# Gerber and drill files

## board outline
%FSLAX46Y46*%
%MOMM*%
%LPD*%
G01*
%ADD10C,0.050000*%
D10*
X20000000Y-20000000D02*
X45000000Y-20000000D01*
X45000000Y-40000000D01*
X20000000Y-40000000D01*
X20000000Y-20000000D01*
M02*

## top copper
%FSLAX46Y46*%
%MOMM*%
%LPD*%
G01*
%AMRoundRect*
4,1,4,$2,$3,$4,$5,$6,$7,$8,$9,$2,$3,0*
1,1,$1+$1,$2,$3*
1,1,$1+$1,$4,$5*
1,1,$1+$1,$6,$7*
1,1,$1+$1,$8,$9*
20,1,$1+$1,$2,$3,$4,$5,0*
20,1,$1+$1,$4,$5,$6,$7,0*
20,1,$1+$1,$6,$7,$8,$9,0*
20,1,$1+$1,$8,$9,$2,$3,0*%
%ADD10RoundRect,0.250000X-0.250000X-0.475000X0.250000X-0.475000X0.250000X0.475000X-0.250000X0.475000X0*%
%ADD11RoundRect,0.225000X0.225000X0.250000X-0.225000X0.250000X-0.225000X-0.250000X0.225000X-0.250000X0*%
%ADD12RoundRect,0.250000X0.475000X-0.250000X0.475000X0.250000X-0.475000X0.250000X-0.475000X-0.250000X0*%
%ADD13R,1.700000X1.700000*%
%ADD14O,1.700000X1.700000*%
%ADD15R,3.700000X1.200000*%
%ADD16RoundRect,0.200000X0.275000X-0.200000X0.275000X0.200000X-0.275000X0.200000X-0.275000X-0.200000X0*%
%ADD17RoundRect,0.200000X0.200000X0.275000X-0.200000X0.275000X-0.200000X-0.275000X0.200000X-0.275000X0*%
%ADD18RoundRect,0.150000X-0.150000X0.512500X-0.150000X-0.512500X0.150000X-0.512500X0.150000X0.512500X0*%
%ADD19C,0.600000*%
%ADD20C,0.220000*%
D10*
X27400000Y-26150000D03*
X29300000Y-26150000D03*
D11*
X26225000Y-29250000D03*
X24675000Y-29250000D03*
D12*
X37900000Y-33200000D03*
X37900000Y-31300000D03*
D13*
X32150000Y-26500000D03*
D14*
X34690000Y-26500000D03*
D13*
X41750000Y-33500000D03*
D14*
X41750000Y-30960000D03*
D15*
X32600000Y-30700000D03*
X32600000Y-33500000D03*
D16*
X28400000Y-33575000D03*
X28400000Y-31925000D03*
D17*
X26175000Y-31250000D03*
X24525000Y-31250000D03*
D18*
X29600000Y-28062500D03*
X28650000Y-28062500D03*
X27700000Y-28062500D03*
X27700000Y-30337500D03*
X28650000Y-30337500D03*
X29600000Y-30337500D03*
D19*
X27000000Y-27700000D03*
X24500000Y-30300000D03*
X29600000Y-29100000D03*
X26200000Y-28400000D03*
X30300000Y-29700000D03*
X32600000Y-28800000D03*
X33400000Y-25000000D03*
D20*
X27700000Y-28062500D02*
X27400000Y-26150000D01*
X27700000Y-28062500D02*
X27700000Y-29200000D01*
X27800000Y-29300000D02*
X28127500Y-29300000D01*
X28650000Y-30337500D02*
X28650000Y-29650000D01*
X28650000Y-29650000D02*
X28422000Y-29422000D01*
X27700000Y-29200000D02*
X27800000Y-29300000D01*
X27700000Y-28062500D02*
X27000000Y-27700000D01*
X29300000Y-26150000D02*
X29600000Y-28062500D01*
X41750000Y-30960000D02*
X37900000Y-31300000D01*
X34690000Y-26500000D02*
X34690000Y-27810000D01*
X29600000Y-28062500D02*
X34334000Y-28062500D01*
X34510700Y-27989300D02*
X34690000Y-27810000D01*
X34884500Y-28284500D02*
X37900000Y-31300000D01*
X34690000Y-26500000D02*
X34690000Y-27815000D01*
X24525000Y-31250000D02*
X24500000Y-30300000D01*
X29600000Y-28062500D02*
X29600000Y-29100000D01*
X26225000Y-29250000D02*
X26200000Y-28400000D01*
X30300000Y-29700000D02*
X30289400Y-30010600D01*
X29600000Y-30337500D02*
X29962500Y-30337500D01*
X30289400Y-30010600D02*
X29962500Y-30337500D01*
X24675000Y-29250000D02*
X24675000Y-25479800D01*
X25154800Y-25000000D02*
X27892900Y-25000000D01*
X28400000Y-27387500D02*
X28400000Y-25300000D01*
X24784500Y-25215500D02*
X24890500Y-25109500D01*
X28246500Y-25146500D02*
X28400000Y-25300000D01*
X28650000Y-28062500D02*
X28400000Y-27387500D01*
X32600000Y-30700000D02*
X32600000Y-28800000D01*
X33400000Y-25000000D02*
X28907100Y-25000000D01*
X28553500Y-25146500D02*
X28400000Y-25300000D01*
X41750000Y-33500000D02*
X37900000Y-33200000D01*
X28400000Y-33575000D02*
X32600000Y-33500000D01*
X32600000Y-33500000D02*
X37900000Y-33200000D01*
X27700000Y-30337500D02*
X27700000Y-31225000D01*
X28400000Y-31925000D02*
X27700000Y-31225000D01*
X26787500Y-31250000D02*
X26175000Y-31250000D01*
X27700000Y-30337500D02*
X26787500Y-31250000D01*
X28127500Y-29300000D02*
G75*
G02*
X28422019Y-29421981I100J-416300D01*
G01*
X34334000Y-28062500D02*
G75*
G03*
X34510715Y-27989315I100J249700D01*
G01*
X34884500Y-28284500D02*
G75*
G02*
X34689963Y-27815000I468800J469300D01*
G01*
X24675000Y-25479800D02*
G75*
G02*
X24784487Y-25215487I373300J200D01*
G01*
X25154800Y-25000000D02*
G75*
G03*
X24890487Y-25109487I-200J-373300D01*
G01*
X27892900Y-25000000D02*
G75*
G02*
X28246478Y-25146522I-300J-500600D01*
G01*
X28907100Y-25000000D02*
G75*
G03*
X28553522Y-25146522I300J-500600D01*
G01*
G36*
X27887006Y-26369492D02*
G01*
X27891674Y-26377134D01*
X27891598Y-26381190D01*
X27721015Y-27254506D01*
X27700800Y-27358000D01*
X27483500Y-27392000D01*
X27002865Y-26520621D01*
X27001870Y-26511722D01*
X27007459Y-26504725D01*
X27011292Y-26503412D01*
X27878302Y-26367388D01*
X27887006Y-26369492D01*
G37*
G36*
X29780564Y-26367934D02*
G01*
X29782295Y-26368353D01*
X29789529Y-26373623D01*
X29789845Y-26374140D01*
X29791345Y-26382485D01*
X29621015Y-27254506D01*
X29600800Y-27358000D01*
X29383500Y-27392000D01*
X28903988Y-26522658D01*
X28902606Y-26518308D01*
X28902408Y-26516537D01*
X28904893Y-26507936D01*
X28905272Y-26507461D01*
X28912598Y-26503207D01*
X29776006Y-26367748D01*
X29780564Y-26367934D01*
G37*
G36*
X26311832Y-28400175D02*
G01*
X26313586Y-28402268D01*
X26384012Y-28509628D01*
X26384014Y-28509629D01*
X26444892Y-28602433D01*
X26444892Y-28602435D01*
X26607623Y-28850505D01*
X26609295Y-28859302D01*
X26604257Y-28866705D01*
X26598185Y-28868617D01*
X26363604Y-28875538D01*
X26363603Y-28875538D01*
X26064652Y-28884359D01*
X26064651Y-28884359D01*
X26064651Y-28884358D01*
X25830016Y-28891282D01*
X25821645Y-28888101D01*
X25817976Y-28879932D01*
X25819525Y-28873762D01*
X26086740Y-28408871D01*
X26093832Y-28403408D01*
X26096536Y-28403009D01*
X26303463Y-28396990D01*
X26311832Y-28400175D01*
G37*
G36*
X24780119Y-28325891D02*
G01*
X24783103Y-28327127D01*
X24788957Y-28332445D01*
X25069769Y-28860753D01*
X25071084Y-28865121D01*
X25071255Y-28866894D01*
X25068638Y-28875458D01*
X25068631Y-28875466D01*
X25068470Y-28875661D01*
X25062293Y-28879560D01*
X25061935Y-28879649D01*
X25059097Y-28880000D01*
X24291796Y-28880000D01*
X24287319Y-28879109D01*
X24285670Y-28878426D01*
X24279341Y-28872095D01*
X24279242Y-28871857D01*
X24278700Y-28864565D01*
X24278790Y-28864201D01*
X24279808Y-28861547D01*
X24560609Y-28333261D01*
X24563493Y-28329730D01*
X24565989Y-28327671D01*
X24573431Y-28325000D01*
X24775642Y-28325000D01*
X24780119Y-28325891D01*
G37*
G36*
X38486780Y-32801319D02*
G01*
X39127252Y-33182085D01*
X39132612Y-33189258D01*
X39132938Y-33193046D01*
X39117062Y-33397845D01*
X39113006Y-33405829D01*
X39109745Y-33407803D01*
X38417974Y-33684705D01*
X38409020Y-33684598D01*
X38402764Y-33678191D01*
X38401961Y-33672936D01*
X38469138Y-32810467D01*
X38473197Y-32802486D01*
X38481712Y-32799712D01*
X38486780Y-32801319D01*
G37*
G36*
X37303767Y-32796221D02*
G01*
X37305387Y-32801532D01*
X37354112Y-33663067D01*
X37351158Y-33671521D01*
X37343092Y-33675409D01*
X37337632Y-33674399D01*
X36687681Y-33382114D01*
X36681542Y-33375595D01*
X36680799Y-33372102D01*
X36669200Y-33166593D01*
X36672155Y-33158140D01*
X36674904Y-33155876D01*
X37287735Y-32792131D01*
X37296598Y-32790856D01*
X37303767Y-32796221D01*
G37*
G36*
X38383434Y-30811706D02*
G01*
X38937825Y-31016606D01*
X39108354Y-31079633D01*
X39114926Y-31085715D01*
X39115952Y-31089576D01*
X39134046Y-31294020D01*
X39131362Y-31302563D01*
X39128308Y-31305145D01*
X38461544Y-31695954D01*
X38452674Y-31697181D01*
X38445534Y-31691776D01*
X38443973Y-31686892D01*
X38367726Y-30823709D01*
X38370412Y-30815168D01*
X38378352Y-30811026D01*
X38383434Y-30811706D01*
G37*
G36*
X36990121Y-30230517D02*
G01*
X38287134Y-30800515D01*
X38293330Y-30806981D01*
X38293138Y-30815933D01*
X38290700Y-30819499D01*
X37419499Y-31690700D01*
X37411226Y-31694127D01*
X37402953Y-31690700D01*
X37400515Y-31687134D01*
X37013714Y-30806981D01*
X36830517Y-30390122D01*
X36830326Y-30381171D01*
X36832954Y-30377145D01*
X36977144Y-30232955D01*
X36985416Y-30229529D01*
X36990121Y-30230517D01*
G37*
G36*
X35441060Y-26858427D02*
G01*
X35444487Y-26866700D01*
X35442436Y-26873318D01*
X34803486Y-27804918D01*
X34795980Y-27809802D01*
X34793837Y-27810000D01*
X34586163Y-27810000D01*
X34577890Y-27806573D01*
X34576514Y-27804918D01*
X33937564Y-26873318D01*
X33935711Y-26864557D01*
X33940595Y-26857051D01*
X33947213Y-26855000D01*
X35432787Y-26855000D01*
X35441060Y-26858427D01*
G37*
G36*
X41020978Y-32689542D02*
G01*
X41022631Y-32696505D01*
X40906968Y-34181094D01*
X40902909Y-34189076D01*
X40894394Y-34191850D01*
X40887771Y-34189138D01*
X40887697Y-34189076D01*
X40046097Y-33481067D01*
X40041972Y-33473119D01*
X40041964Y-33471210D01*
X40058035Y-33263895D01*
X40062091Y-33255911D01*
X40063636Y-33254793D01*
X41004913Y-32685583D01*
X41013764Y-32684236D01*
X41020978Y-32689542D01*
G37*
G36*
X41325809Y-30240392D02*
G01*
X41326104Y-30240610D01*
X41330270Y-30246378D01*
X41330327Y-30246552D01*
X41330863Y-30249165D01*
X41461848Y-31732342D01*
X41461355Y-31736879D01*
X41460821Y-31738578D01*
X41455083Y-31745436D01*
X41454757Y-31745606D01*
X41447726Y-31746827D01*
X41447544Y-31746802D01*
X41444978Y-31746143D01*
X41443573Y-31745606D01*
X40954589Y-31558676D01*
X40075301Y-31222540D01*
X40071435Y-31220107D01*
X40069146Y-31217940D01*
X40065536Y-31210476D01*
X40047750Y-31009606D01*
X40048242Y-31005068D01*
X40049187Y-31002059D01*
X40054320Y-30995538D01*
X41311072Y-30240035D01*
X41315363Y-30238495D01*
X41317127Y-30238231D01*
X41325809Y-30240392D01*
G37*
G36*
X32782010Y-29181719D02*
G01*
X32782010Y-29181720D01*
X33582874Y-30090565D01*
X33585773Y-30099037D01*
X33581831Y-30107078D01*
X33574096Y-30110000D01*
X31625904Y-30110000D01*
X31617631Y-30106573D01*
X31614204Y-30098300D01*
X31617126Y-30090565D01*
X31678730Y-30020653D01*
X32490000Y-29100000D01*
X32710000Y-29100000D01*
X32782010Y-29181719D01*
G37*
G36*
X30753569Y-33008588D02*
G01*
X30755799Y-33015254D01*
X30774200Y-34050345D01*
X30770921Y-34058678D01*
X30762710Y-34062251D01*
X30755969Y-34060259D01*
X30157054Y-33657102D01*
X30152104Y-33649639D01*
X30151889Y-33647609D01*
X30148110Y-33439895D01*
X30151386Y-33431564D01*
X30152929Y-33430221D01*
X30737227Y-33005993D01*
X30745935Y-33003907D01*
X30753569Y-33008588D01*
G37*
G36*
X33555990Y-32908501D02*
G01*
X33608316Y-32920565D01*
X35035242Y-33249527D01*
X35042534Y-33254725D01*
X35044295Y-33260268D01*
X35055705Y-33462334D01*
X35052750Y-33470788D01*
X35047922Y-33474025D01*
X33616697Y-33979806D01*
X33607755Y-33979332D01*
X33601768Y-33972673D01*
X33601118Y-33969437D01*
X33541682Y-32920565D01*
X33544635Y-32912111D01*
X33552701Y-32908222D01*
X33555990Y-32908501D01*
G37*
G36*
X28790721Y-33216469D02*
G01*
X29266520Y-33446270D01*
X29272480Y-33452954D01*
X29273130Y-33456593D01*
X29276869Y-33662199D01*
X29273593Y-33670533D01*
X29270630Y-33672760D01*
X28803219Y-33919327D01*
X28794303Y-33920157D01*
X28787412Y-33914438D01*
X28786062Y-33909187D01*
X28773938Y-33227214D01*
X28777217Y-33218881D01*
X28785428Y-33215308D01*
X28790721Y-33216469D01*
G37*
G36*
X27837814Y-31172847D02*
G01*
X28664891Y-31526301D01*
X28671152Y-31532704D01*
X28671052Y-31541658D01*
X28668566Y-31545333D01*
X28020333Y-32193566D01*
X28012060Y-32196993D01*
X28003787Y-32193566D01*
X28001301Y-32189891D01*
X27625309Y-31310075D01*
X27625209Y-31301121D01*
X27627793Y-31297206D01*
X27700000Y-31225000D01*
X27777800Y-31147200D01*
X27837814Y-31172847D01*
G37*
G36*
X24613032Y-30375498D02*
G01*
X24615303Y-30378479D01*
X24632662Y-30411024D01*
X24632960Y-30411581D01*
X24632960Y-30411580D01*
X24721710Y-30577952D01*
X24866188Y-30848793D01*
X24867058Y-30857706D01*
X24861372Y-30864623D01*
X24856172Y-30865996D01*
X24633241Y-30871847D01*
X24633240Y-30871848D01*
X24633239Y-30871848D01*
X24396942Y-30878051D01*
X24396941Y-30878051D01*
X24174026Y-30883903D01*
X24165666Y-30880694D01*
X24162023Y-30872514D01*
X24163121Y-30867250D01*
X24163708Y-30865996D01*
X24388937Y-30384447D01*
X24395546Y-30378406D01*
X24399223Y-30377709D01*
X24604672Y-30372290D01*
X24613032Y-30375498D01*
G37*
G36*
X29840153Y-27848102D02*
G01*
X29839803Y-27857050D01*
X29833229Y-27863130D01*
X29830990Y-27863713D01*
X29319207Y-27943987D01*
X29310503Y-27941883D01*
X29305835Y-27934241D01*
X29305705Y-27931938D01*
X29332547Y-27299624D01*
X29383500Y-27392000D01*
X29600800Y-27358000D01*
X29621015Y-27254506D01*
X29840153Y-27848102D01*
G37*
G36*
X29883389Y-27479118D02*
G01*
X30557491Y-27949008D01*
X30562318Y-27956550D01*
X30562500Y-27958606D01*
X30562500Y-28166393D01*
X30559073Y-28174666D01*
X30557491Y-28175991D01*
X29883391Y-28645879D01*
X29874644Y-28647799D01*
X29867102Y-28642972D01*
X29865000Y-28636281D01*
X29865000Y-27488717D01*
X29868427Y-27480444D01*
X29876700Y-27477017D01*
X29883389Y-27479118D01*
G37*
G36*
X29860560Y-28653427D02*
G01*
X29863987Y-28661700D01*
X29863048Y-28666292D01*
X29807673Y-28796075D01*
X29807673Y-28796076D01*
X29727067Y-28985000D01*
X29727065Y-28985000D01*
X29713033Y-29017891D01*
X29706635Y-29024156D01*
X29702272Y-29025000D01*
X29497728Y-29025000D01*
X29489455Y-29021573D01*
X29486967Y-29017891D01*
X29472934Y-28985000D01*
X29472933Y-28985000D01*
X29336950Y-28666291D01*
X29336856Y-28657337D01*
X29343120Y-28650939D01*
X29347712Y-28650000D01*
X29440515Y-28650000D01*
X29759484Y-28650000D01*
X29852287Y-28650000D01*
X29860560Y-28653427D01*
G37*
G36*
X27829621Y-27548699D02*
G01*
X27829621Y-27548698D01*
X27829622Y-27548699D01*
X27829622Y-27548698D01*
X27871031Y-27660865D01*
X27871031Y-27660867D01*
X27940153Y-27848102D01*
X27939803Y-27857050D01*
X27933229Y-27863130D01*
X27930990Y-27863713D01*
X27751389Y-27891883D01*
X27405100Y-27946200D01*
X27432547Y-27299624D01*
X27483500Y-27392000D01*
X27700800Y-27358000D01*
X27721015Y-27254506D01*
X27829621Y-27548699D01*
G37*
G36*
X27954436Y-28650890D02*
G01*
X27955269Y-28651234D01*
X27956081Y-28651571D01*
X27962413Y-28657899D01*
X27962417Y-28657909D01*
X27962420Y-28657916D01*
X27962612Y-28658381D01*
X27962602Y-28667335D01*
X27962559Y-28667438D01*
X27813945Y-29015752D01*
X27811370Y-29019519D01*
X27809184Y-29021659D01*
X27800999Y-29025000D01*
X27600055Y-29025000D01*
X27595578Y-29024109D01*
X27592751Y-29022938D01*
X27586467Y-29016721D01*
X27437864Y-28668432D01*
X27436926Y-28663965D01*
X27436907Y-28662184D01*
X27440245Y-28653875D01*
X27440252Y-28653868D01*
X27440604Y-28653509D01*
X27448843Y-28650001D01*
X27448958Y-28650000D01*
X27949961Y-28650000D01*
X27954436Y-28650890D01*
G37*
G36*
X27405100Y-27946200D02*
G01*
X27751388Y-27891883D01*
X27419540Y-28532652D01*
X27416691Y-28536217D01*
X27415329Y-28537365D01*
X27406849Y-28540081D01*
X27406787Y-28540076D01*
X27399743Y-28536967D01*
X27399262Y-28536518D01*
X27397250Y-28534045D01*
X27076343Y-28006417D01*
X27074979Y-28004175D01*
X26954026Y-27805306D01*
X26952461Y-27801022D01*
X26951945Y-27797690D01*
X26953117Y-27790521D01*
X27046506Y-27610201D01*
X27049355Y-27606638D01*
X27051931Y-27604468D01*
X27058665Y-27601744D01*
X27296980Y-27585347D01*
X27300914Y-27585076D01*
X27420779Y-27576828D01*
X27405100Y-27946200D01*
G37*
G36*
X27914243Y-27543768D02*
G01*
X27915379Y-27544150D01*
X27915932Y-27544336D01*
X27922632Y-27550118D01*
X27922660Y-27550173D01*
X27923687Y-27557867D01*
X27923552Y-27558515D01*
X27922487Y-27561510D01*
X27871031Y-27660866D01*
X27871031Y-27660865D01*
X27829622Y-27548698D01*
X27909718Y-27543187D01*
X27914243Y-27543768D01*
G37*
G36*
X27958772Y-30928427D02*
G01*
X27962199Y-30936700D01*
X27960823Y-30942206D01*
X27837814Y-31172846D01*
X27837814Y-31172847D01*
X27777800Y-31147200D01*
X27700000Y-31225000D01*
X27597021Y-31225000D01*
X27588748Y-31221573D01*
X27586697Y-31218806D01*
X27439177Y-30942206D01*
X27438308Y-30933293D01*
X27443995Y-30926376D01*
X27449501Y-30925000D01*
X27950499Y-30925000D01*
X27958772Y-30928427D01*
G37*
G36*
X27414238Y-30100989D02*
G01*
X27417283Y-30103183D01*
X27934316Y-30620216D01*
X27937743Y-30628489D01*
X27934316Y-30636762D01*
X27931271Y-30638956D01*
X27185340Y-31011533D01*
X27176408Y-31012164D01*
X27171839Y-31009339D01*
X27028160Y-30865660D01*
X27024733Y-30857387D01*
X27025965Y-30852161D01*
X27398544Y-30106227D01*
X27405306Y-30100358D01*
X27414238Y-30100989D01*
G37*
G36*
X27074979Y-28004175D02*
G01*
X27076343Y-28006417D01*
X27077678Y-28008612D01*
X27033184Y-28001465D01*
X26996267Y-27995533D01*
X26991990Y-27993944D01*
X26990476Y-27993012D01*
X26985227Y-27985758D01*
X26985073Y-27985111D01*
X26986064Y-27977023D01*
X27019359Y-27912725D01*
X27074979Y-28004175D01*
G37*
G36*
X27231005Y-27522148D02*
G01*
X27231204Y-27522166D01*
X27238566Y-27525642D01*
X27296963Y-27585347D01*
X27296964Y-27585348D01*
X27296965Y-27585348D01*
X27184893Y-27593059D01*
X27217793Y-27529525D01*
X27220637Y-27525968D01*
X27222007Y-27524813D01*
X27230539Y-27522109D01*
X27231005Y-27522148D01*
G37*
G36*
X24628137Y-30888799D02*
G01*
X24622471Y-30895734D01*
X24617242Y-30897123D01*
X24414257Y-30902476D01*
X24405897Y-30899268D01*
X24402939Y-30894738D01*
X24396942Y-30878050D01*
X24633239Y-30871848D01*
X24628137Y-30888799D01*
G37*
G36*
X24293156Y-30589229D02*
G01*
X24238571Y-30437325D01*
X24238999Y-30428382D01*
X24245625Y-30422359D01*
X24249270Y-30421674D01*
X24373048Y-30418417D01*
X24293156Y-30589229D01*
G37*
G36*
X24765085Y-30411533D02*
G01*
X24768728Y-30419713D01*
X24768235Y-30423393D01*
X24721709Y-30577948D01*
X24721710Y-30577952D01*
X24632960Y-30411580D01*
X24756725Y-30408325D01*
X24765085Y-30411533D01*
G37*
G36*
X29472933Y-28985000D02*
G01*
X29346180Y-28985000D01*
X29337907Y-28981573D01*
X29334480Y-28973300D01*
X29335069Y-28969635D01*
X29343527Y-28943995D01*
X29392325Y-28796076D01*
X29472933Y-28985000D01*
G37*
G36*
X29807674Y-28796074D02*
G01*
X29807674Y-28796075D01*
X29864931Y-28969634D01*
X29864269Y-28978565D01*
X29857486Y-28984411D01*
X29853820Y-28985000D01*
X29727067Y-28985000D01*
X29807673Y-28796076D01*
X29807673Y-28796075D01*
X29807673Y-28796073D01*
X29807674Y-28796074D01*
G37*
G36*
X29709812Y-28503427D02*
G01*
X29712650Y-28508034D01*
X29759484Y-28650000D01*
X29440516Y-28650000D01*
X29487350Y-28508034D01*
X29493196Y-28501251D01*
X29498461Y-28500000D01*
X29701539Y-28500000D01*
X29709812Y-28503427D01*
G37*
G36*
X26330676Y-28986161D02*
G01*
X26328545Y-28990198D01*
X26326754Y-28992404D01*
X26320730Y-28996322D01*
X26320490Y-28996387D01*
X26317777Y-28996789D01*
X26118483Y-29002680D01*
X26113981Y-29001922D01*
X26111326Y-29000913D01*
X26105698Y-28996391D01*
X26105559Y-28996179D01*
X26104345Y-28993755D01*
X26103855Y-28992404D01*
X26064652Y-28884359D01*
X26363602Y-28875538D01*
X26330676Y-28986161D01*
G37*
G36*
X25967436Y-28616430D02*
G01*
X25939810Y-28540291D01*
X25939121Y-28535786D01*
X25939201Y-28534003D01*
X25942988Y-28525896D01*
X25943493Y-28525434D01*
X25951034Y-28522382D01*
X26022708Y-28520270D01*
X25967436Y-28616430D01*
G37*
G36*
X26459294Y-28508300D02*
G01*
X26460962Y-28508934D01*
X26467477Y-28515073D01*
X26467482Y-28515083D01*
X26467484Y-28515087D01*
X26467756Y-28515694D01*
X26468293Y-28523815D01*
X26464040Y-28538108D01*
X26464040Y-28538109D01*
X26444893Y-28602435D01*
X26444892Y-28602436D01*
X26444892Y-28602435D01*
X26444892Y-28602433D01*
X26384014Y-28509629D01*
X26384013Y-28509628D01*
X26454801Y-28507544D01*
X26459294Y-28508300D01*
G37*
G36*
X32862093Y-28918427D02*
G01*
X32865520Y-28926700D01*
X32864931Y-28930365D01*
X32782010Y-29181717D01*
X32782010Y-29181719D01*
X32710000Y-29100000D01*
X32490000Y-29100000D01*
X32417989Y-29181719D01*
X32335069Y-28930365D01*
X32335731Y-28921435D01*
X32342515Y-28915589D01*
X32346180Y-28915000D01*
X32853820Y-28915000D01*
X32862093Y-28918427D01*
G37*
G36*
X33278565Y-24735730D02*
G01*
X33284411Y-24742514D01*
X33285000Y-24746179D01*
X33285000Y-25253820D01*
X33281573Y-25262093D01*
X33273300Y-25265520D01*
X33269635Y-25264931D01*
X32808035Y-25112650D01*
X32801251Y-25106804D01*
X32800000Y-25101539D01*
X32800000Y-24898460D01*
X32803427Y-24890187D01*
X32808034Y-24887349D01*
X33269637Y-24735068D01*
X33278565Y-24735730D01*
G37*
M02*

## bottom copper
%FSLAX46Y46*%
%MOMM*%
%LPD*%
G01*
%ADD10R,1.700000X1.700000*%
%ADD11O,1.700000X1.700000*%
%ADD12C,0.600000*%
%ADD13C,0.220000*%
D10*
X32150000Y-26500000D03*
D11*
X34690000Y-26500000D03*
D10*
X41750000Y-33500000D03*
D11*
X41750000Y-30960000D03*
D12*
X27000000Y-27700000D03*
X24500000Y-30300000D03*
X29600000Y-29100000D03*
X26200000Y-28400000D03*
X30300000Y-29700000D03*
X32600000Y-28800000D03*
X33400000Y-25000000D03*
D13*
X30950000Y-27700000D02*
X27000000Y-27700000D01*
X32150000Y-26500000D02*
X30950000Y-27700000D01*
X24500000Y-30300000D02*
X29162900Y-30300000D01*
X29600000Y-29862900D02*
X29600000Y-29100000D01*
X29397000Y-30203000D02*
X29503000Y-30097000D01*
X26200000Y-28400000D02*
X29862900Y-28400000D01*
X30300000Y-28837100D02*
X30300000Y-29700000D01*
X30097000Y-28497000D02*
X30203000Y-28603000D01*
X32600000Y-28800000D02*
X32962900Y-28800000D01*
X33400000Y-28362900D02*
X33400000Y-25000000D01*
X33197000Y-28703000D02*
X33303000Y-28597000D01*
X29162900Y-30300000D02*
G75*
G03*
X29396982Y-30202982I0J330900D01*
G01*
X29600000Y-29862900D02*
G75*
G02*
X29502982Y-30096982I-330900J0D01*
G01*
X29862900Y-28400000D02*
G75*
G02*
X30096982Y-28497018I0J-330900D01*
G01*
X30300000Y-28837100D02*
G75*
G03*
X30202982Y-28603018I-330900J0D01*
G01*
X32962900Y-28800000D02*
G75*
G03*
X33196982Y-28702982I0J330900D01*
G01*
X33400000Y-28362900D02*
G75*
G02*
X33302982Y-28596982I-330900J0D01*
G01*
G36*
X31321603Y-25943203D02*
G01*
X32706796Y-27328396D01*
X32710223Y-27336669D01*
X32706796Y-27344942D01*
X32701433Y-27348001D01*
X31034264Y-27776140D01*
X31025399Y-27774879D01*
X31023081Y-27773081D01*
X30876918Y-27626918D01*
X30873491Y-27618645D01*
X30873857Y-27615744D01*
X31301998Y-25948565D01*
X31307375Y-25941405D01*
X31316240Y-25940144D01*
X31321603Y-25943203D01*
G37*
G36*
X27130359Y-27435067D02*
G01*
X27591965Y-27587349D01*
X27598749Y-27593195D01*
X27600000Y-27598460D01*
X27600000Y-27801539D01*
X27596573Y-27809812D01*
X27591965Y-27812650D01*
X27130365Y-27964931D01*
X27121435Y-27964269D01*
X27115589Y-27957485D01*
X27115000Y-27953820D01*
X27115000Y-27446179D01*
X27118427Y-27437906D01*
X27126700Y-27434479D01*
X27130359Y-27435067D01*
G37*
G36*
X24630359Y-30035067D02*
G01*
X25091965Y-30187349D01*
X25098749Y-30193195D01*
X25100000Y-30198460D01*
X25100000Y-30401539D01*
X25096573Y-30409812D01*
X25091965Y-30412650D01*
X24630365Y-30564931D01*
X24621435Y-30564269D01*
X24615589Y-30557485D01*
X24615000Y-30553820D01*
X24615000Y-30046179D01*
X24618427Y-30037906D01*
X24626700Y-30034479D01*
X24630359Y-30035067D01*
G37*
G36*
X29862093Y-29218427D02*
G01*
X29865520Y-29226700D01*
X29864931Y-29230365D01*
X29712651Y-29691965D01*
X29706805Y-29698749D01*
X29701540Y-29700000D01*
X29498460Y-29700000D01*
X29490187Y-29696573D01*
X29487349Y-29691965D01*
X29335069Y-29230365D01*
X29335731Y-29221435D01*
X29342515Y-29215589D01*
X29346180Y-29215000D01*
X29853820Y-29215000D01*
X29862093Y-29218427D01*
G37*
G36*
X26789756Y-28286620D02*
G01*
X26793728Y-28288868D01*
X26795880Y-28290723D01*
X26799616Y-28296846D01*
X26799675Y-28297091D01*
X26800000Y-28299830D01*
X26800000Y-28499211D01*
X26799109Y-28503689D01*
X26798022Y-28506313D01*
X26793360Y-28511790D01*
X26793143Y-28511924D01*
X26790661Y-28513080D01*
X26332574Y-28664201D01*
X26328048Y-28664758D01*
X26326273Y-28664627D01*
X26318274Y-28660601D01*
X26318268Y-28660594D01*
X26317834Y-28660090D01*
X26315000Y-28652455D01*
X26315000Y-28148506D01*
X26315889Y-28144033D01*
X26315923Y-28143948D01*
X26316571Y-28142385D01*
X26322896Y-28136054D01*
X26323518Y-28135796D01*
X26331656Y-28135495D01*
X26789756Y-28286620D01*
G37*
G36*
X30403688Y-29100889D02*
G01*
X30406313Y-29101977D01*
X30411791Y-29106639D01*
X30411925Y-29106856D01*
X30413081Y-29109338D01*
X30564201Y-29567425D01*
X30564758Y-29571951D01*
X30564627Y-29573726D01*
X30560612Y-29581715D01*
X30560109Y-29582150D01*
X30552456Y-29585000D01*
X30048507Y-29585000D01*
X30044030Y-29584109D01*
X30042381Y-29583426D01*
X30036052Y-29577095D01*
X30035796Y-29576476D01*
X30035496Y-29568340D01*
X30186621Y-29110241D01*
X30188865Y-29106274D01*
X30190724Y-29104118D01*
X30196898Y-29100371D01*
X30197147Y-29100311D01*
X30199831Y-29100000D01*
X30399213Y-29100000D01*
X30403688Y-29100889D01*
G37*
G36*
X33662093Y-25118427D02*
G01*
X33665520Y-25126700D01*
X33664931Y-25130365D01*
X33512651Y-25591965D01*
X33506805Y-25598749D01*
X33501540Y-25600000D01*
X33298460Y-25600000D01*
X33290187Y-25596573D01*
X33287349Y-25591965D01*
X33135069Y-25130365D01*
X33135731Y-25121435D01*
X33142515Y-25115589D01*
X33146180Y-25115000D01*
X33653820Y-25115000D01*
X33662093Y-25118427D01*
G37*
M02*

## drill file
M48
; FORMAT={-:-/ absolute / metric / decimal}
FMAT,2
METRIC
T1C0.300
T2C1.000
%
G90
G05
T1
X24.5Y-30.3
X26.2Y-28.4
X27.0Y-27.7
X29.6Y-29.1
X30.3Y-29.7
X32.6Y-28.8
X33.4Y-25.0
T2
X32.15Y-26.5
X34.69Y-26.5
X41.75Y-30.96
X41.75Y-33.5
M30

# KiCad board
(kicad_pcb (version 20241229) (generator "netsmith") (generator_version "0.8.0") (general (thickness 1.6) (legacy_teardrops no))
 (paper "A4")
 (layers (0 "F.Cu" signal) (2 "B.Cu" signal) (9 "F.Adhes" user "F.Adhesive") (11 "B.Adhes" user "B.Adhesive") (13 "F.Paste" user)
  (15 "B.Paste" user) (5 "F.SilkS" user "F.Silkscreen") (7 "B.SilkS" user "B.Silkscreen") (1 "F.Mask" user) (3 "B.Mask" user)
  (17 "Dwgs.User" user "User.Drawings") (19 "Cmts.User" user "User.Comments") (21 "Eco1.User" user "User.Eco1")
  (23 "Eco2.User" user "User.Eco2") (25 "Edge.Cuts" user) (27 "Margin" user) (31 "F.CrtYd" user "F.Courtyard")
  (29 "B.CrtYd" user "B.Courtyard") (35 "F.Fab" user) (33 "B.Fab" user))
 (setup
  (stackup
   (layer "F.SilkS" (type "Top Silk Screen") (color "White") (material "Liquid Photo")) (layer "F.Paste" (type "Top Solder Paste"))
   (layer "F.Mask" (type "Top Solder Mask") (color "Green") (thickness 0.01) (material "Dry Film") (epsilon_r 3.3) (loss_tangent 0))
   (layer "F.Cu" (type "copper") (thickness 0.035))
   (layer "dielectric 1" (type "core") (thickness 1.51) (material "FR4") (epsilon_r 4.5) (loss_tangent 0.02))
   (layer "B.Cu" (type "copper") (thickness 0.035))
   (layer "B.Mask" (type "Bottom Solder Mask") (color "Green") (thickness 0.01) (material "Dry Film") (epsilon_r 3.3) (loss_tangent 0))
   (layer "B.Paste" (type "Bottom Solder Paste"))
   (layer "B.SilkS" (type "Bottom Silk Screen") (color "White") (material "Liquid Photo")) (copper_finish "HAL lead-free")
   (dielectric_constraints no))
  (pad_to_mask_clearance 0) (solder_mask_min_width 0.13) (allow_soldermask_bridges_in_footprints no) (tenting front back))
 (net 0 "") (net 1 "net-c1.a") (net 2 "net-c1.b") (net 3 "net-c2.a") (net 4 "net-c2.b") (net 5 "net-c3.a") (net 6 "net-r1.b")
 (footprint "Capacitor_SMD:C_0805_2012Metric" (layer "F.Cu") (at 28.35 26.15)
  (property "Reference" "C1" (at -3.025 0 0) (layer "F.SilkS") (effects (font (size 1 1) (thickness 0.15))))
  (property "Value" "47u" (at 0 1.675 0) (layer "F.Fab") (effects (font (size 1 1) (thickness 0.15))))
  (pad "1" smd roundrect (at -0.95 0) (size 1 1.45) (layers "F.Cu" "F.Mask" "F.Paste") (roundrect_rratio 0.25) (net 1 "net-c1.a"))
  (pad "2" smd roundrect (at 0.95 0) (size 1 1.45) (layers "F.Cu" "F.Mask" "F.Paste") (roundrect_rratio 0.25) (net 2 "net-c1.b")))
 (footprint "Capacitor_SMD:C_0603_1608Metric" (layer "F.Cu") (at 25.45 29.25 180)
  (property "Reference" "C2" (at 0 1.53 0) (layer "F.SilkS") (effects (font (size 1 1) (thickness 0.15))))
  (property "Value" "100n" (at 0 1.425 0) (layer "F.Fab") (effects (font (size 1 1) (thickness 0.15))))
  (pad "1" smd roundrect (at -0.775 0 180) (size 0.9 0.95) (layers "F.Cu" "F.Mask" "F.Paste") (roundrect_rratio 0.25) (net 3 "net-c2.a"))
  (pad "2" smd roundrect (at 0.775 0 180) (size 0.9 0.95) (layers "F.Cu" "F.Mask" "F.Paste") (roundrect_rratio 0.25) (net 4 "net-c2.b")))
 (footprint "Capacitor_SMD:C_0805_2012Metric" (layer "F.Cu") (at 37.9 32.25 90)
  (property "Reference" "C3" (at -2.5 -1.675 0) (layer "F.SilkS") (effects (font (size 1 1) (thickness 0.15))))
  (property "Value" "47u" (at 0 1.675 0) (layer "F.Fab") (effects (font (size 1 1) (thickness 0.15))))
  (pad "1" smd roundrect (at -0.95 0 90) (size 1 1.45) (layers "F.Cu" "F.Mask" "F.Paste") (roundrect_rratio 0.25) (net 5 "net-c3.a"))
  (pad "2" smd roundrect (at 0.95 0 90) (size 1 1.45) (layers "F.Cu" "F.Mask" "F.Paste") (roundrect_rratio 0.25) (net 2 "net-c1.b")))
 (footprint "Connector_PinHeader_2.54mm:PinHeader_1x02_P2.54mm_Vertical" (layer "F.Cu") (at 32.15 26.5 90)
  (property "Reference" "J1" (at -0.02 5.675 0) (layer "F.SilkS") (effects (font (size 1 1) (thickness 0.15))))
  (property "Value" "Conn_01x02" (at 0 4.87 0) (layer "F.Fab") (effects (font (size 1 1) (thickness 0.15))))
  (pad "1" thru_hole rect (at 0 0 90) (size 1.7 1.7) (drill 1) (layers "*.Cu" "*.Mask") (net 1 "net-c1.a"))
  (pad "2" thru_hole oval (at 0 2.54 90) (size 1.7 1.7) (drill 1) (layers "*.Cu" "*.Mask") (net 2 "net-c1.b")))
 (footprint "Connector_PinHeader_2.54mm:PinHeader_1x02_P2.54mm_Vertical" (layer "F.Cu") (at 41.75 33.5 180)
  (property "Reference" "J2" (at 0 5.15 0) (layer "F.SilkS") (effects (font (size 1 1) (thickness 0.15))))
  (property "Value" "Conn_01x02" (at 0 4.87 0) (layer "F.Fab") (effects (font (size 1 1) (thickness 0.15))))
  (pad "1" thru_hole rect (at 0 0 180) (size 1.7 1.7) (drill 1) (layers "*.Cu" "*.Mask") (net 5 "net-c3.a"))
  (pad "2" thru_hole oval (at 0 2.54 180) (size 1.7 1.7) (drill 1) (layers "*.Cu" "*.Mask") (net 2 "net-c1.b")))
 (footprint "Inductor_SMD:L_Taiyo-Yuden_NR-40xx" (layer "F.Cu") (at 32.6 32.1 270)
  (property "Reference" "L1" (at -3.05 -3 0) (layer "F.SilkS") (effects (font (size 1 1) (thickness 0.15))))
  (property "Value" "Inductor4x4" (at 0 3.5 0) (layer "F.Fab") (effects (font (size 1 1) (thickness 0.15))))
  (pad "1" smd rect (at -1.4 0 270) (size 1.2 3.7) (layers "F.Cu" "F.Mask" "F.Paste") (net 4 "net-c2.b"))
  (pad "2" smd rect (at 1.4 0 270) (size 1.2 3.7) (layers "F.Cu" "F.Mask" "F.Paste") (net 5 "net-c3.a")))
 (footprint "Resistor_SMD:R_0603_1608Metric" (layer "F.Cu") (at 28.4 32.75 90)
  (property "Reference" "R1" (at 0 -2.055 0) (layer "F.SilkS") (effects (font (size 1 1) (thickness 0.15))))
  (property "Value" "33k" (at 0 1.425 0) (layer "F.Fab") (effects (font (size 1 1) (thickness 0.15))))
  (pad "1" smd roundrect (at -0.825 0 90) (size 0.8 0.95) (layers "F.Cu" "F.Mask" "F.Paste") (roundrect_rratio 0.25) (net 5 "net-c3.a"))
  (pad "2" smd roundrect (at 0.825 0 90) (size 0.8 0.95) (layers "F.Cu" "F.Mask" "F.Paste") (roundrect_rratio 0.25) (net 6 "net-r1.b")))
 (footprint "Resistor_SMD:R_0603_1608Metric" (layer "F.Cu") (at 25.35 31.25 180)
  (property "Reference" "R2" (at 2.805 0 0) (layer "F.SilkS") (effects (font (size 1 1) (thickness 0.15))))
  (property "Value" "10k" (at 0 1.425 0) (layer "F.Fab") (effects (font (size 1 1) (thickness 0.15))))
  (pad "1" smd roundrect (at -0.825 0 180) (size 0.8 0.95) (layers "F.Cu" "F.Mask" "F.Paste") (roundrect_rratio 0.25) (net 6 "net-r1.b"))
  (pad "2" smd roundrect (at 0.825 0 180) (size 0.8 0.95) (layers "F.Cu" "F.Mask" "F.Paste") (roundrect_rratio 0.25) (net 2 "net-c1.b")))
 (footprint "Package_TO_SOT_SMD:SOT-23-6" (layer "F.Cu") (at 28.65 29.2 270)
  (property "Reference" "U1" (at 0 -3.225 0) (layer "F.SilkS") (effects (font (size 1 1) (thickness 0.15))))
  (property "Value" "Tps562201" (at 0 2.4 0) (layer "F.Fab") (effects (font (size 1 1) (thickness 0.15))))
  (pad "1" smd roundrect (at -1.1375 -0.95 270) (size 1.325 0.6) (layers "F.Cu" "F.Mask" "F.Paste") (roundrect_rratio 0.25)
   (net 2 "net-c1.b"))
  (pad "2" smd roundrect (at -1.1375 0 270) (size 1.325 0.6) (layers "F.Cu" "F.Mask" "F.Paste") (roundrect_rratio 0.25) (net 4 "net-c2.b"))
  (pad "3" smd roundrect (at -1.1375 0.95 270) (size 1.325 0.6) (layers "F.Cu" "F.Mask" "F.Paste") (roundrect_rratio 0.25)
   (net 1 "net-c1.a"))
  (pad "4" smd roundrect (at 1.1375 0.95 270) (size 1.325 0.6) (layers "F.Cu" "F.Mask" "F.Paste") (roundrect_rratio 0.25) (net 6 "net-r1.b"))
  (pad "5" smd roundrect (at 1.1375 0 270) (size 1.325 0.6) (layers "F.Cu" "F.Mask" "F.Paste") (roundrect_rratio 0.25) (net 1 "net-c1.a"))
  (pad "6" smd roundrect (at 1.1375 -0.95 270) (size 1.325 0.6) (layers "F.Cu" "F.Mask" "F.Paste") (roundrect_rratio 0.25)
   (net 3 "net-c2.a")))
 (segment (start 27.7 28.0625) (end 27.4 26.15) (width 0.22) (layer "F.Cu") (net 1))
 (segment (start 27.7 28.0625) (end 27.7 29.2) (width 0.22) (layer "F.Cu") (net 1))
 (segment (start 27.8 29.3) (end 28.1275 29.3) (width 0.22) (layer "F.Cu") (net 1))
 (segment (start 28.65 30.3375) (end 28.65 29.65) (width 0.22) (layer "F.Cu") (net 1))
 (segment (start 28.65 29.65) (end 28.422 29.422) (width 0.22) (layer "F.Cu") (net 1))
 (segment (start 27.7 29.2) (end 27.8 29.3) (width 0.22) (layer "F.Cu") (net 1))
 (segment (start 30.95 27.7) (end 27 27.7) (width 0.22) (layer "B.Cu") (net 1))
 (segment (start 27.7 28.0625) (end 27 27.7) (width 0.22) (layer "F.Cu") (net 1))
 (segment (start 32.15 26.5) (end 30.95 27.7) (width 0.22) (layer "B.Cu") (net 1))
 (segment (start 29.3 26.15) (end 29.6 28.0625) (width 0.22) (layer "F.Cu") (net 2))
 (segment (start 41.75 30.96) (end 37.9 31.3) (width 0.22) (layer "F.Cu") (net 2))
 (segment (start 34.69 26.5) (end 34.69 27.81) (width 0.22) (layer "F.Cu") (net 2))
 (segment (start 29.6 28.0625) (end 34.334 28.0625) (width 0.22) (layer "F.Cu") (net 2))
 (segment (start 34.5107 27.9893) (end 34.69 27.81) (width 0.22) (layer "F.Cu") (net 2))
 (segment (start 34.8845 28.2845) (end 37.9 31.3) (width 0.22) (layer "F.Cu") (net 2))
 (segment (start 34.69 26.5) (end 34.69 27.815) (width 0.22) (layer "F.Cu") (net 2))
 (segment (start 24.525 31.25) (end 24.5 30.3) (width 0.22) (layer "F.Cu") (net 2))
 (segment (start 24.5 30.3) (end 29.1629 30.3) (width 0.22) (layer "B.Cu") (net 2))
 (segment (start 29.6 29.8629) (end 29.6 29.1) (width 0.22) (layer "B.Cu") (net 2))
 (segment (start 29.6 28.0625) (end 29.6 29.1) (width 0.22) (layer "F.Cu") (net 2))
 (segment (start 29.397 30.203) (end 29.503 30.097) (width 0.22) (layer "B.Cu") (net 2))
 (segment (start 26.225 29.25) (end 26.2 28.4) (width 0.22) (layer "F.Cu") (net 3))
 (segment (start 26.2 28.4) (end 29.8629 28.4) (width 0.22) (layer "B.Cu") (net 3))
 (segment (start 30.3 28.8371) (end 30.3 29.7) (width 0.22) (layer "B.Cu") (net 3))
 (segment (start 30.3 29.7) (end 30.2894 30.0106) (width 0.22) (layer "F.Cu") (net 3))
 (segment (start 29.6 30.3375) (end 29.9625 30.3375) (width 0.22) (layer "F.Cu") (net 3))
 (segment (start 30.097 28.497) (end 30.203 28.603) (width 0.22) (layer "B.Cu") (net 3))
 (segment (start 30.2894 30.0106) (end 29.9625 30.3375) (width 0.22) (layer "F.Cu") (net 3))
 (segment (start 24.675 29.25) (end 24.675 25.4798) (width 0.22) (layer "F.Cu") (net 4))
 (segment (start 25.1548 25) (end 27.8929 25) (width 0.22) (layer "F.Cu") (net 4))
 (segment (start 28.4 27.3875) (end 28.4 25.3) (width 0.22) (layer "F.Cu") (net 4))
 (segment (start 24.7845 25.2155) (end 24.8905 25.1095) (width 0.22) (layer "F.Cu") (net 4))
 (segment (start 28.2465 25.1465) (end 28.4 25.3) (width 0.22) (layer "F.Cu") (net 4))
 (segment (start 28.65 28.0625) (end 28.4 27.3875) (width 0.22) (layer "F.Cu") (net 4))
 (segment (start 32.6 30.7) (end 32.6 28.8) (width 0.22) (layer "F.Cu") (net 4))
 (segment (start 32.6 28.8) (end 32.9629 28.8) (width 0.22) (layer "B.Cu") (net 4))
 (segment (start 33.4 28.3629) (end 33.4 25) (width 0.22) (layer "B.Cu") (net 4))
 (segment (start 33.4 25) (end 28.9071 25) (width 0.22) (layer "F.Cu") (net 4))
 (segment (start 33.197 28.703) (end 33.303 28.597) (width 0.22) (layer "B.Cu") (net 4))
 (segment (start 28.5535 25.1465) (end 28.4 25.3) (width 0.22) (layer "F.Cu") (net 4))
 (segment (start 41.75 33.5) (end 37.9 33.2) (width 0.22) (layer "F.Cu") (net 5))
 (segment (start 28.4 33.575) (end 32.6 33.5) (width 0.22) (layer "F.Cu") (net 5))
 (segment (start 32.6 33.5) (end 37.9 33.2) (width 0.22) (layer "F.Cu") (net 5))
 (segment (start 27.7 30.3375) (end 27.7 31.225) (width 0.22) (layer "F.Cu") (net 6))
 (segment (start 28.4 31.925) (end 27.7 31.225) (width 0.22) (layer "F.Cu") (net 6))
 (segment (start 26.7875 31.25) (end 26.175 31.25) (width 0.22) (layer "F.Cu") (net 6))
 (segment (start 27.7 30.3375) (end 26.7875 31.25) (width 0.22) (layer "F.Cu") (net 6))
 (arc (start 28.1275 29.3) (mid 28.2869 29.3317) (end 28.422 29.422) (width 0.22) (layer "F.Cu") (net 1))
 (arc (start 34.334 28.0625) (mid 34.4296 28.0435) (end 34.5107 27.9893) (width 0.22) (layer "F.Cu") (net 2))
 (arc (start 34.8845 28.2845) (mid 34.7405 28.0691) (end 34.69 27.815) (width 0.22) (layer "F.Cu") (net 2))
 (arc (start 29.1629 30.3) (mid 29.2896 30.2748) (end 29.397 30.203) (width 0.22) (layer "B.Cu") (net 2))
 (arc (start 29.6 29.8629) (mid 29.5748 29.9896) (end 29.503 30.097) (width 0.22) (layer "B.Cu") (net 2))
 (arc (start 29.8629 28.4) (mid 29.9896 28.4252) (end 30.097 28.497) (width 0.22) (layer "B.Cu") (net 3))
 (arc (start 30.3 28.8371) (mid 30.2748 28.7104) (end 30.203 28.603) (width 0.22) (layer "B.Cu") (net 3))
 (arc (start 24.675 25.4798) (mid 24.7034 25.3368) (end 24.7845 25.2155) (width 0.22) (layer "F.Cu") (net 4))
 (arc (start 25.1548 25) (mid 25.0118 25.0284) (end 24.8905 25.1095) (width 0.22) (layer "F.Cu") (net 4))
 (arc (start 27.8929 25) (mid 28.0842 25.0381) (end 28.2465 25.1465) (width 0.22) (layer "F.Cu") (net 4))
 (arc (start 32.9629 28.8) (mid 33.0896 28.7748) (end 33.197 28.703) (width 0.22) (layer "B.Cu") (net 4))
 (arc (start 33.4 28.3629) (mid 33.3748 28.4896) (end 33.303 28.597) (width 0.22) (layer "B.Cu") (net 4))
 (arc (start 28.9071 25) (mid 28.7158 25.0381) (end 28.5535 25.1465) (width 0.22) (layer "F.Cu") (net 4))
 (via (at 27 27.7) (size 0.6) (drill 0.3) (layers "F.Cu" "B.Cu") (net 1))
 (via (at 24.5 30.3) (size 0.6) (drill 0.3) (layers "F.Cu" "B.Cu") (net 2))
 (via (at 29.6 29.1) (size 0.6) (drill 0.3) (layers "F.Cu" "B.Cu") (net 2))
 (via (at 26.2 28.4) (size 0.6) (drill 0.3) (layers "F.Cu" "B.Cu") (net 3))
 (via (at 30.3 29.7) (size 0.6) (drill 0.3) (layers "F.Cu" "B.Cu") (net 3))
 (via (at 32.6 28.8) (size 0.6) (drill 0.3) (layers "F.Cu" "B.Cu") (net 4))
 (via (at 33.4 25) (size 0.6) (drill 0.3) (layers "F.Cu" "B.Cu") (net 4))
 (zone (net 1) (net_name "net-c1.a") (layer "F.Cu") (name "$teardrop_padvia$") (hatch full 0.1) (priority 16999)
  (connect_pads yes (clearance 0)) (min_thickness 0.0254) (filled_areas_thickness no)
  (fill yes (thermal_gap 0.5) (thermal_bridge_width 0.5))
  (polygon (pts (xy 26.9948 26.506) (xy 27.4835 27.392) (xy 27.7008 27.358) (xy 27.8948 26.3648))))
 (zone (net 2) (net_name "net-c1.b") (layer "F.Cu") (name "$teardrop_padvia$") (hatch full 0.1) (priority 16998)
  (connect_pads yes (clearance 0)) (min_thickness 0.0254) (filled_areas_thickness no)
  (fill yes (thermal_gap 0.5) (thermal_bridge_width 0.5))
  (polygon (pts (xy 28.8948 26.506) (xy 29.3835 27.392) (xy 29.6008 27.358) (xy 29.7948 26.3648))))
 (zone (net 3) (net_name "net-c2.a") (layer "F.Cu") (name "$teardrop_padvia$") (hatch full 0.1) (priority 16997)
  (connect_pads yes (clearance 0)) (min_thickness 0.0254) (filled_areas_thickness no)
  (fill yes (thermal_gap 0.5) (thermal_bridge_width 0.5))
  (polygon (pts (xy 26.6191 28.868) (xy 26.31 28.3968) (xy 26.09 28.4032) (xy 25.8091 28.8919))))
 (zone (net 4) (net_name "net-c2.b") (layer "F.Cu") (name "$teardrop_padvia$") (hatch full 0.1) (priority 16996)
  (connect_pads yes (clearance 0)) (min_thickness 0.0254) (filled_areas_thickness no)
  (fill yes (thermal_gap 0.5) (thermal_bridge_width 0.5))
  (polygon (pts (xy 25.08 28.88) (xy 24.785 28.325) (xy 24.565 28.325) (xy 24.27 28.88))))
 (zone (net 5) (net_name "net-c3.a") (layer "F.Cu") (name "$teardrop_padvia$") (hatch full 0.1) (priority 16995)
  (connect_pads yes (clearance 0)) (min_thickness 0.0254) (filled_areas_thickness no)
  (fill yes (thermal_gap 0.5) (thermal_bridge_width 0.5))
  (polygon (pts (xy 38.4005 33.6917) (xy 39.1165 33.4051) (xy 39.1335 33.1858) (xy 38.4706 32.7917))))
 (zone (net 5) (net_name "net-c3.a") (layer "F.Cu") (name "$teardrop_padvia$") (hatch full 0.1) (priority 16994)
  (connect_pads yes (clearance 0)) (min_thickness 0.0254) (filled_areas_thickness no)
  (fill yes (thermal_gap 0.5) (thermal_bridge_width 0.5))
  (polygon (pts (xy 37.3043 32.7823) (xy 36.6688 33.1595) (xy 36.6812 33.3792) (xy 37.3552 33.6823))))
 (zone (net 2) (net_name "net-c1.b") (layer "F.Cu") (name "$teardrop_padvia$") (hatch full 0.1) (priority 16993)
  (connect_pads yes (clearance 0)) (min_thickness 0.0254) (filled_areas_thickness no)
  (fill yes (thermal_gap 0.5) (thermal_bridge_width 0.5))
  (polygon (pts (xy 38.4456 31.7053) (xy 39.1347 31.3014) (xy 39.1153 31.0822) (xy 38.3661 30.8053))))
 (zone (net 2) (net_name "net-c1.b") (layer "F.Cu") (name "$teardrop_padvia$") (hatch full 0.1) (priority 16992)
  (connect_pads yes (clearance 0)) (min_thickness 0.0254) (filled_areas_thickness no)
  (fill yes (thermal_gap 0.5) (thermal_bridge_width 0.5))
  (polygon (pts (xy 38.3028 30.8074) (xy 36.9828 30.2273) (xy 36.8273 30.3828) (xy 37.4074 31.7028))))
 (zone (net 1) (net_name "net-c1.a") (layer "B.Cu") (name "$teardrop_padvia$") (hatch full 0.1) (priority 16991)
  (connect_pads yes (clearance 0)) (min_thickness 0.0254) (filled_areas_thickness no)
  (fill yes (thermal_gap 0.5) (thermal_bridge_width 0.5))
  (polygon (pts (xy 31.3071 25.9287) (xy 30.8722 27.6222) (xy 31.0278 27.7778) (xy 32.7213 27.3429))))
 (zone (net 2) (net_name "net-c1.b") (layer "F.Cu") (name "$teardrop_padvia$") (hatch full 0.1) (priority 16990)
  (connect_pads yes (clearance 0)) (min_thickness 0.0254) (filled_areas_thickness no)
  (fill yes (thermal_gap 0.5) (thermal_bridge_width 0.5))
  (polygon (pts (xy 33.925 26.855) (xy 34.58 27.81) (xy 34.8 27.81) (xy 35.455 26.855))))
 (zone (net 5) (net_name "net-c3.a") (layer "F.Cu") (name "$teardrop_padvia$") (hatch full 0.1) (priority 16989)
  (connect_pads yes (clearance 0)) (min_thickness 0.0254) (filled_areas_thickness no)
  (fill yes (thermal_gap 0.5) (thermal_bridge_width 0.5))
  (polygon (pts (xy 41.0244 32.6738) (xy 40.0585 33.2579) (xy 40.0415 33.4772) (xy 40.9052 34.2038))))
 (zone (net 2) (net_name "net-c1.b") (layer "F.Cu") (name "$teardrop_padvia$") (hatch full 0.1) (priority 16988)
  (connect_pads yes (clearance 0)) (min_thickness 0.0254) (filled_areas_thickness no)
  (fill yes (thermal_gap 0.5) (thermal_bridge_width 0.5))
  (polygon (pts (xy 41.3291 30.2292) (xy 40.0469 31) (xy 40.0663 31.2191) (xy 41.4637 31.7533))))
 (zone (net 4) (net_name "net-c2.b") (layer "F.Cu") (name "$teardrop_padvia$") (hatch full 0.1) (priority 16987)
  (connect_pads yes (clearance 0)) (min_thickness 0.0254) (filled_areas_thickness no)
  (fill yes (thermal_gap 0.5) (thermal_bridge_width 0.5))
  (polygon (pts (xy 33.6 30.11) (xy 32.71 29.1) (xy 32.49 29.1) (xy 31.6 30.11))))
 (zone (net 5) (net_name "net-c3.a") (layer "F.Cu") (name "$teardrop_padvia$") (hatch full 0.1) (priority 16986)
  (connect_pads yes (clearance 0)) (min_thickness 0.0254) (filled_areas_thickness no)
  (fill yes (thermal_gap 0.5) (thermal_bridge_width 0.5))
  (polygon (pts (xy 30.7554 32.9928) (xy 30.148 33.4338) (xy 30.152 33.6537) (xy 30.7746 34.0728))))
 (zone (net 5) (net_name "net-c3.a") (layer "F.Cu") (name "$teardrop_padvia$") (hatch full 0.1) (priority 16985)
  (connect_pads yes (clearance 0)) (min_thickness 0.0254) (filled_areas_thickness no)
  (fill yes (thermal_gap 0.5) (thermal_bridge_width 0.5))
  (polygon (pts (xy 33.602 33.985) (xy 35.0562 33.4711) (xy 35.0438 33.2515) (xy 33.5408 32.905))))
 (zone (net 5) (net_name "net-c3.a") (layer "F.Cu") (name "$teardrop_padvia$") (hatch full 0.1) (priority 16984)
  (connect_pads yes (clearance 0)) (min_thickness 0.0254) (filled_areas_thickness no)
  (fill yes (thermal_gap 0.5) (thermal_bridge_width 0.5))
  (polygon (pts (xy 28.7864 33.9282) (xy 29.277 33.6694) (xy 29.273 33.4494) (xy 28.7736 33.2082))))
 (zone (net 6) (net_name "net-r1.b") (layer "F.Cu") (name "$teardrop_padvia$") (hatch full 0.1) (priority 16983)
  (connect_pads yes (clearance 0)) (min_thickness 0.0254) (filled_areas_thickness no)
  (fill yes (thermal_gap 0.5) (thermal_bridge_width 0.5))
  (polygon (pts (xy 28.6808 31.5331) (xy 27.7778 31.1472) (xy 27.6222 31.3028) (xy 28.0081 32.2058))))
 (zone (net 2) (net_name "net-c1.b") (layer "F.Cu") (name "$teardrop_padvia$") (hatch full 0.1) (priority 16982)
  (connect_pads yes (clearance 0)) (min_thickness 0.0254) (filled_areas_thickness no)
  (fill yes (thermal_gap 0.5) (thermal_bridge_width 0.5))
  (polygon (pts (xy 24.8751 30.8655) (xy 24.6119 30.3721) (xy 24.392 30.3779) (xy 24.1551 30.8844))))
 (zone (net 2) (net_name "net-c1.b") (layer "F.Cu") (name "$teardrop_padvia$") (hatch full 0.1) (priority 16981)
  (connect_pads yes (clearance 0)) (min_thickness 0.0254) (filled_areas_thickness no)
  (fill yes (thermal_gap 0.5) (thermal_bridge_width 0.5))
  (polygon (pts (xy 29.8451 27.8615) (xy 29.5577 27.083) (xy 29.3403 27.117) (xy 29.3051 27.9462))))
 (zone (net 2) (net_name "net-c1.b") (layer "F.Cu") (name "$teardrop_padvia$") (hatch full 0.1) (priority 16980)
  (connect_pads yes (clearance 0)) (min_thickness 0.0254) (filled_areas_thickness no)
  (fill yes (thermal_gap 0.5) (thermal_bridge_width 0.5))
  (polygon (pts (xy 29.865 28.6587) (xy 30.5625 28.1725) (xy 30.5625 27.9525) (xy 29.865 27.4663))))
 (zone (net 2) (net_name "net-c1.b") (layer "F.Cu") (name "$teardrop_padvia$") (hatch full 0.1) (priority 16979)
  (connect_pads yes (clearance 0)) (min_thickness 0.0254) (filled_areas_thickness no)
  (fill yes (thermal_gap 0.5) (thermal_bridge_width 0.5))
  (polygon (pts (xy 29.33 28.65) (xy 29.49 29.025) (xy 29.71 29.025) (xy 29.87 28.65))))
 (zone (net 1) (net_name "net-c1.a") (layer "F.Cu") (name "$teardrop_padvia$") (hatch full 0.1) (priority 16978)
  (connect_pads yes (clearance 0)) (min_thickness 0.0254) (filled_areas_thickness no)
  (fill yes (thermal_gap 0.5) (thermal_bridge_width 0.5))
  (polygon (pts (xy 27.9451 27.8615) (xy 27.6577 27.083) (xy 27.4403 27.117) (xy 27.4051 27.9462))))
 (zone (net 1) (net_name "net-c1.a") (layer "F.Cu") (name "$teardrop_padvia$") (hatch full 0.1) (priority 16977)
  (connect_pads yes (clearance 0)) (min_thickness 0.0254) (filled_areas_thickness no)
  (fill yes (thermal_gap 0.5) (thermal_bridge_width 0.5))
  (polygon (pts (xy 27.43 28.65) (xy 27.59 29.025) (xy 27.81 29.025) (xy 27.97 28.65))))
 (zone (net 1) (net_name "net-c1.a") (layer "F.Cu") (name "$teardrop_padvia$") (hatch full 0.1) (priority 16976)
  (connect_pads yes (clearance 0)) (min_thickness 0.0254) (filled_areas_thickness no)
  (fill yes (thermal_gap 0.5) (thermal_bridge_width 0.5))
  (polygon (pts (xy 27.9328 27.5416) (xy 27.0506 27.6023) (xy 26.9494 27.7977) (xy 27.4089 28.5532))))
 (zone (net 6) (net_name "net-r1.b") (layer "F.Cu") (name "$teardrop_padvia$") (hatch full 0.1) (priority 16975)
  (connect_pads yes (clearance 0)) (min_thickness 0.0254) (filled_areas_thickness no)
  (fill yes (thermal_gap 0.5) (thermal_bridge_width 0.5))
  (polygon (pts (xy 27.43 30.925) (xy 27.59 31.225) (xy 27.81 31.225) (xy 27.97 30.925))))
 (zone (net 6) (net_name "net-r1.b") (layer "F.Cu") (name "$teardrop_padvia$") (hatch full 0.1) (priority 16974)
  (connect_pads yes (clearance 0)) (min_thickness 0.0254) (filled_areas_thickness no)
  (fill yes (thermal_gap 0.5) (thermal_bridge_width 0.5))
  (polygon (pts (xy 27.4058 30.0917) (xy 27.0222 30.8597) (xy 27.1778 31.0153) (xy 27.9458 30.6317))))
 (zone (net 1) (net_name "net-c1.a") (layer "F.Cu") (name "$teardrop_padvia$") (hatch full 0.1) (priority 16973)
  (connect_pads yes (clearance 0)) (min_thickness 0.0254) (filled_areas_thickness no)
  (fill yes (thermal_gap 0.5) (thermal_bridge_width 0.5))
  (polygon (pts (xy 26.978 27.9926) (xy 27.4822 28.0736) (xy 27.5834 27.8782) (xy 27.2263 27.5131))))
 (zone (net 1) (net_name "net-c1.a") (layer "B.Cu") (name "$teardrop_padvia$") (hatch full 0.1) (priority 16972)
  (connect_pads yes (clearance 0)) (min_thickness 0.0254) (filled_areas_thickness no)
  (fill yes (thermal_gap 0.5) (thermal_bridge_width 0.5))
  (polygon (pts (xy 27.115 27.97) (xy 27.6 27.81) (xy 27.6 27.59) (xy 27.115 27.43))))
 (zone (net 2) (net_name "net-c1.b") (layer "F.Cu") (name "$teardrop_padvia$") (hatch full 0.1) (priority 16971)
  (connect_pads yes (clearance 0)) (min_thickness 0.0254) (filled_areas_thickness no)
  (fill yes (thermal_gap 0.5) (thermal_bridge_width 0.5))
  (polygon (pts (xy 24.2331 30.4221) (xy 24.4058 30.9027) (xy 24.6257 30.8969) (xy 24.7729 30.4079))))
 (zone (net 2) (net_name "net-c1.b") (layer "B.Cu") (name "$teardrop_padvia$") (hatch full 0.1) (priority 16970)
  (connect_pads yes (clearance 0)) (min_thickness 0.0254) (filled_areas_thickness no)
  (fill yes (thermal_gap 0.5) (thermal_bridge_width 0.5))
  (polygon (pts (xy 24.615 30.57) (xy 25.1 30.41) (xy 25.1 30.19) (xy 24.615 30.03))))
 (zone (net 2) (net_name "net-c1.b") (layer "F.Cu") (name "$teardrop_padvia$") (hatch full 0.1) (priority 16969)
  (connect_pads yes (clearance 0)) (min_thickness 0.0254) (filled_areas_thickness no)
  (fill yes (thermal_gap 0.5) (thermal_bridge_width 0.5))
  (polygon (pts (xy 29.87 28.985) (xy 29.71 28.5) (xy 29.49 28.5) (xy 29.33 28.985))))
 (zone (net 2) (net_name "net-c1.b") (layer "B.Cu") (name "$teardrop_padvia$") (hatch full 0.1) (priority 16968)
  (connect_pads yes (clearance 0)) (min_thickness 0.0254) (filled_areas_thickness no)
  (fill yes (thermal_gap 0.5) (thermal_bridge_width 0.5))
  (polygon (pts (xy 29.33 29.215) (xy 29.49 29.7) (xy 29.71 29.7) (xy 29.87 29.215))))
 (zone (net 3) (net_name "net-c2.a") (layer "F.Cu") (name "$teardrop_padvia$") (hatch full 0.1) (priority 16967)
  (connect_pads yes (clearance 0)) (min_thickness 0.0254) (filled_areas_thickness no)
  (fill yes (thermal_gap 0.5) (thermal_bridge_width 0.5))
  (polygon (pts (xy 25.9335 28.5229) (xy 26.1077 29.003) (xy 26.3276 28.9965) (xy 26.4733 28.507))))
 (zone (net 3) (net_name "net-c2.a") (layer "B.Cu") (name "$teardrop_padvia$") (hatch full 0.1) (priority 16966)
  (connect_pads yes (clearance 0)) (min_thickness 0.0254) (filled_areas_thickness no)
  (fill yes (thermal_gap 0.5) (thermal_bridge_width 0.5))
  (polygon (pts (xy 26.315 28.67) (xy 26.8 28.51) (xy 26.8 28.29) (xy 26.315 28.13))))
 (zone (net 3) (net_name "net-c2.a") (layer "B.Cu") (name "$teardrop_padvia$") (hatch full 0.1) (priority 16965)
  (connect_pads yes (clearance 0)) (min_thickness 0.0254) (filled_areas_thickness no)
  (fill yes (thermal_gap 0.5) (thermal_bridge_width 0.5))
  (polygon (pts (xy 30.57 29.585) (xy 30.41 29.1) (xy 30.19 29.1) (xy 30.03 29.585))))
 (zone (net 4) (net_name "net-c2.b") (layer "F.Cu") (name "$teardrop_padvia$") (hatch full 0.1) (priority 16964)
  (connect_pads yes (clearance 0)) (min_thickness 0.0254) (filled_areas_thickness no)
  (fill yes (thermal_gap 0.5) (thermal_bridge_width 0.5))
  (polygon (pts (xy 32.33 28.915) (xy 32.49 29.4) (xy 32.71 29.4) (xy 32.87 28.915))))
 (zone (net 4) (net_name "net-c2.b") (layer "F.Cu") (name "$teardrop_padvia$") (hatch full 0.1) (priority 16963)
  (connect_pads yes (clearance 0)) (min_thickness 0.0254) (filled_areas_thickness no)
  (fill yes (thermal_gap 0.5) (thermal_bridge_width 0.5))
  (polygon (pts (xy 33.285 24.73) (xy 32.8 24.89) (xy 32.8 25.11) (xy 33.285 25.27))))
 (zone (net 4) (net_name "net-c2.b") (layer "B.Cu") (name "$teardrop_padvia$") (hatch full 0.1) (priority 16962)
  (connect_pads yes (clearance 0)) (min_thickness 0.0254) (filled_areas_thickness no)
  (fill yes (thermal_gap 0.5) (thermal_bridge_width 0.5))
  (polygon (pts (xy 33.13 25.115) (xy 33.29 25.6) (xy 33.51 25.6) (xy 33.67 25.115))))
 (gr_rect (start 20 20) (end 45 40) (stroke (width 0.05) (type default)) (fill no) (layer "Edge.Cuts")))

